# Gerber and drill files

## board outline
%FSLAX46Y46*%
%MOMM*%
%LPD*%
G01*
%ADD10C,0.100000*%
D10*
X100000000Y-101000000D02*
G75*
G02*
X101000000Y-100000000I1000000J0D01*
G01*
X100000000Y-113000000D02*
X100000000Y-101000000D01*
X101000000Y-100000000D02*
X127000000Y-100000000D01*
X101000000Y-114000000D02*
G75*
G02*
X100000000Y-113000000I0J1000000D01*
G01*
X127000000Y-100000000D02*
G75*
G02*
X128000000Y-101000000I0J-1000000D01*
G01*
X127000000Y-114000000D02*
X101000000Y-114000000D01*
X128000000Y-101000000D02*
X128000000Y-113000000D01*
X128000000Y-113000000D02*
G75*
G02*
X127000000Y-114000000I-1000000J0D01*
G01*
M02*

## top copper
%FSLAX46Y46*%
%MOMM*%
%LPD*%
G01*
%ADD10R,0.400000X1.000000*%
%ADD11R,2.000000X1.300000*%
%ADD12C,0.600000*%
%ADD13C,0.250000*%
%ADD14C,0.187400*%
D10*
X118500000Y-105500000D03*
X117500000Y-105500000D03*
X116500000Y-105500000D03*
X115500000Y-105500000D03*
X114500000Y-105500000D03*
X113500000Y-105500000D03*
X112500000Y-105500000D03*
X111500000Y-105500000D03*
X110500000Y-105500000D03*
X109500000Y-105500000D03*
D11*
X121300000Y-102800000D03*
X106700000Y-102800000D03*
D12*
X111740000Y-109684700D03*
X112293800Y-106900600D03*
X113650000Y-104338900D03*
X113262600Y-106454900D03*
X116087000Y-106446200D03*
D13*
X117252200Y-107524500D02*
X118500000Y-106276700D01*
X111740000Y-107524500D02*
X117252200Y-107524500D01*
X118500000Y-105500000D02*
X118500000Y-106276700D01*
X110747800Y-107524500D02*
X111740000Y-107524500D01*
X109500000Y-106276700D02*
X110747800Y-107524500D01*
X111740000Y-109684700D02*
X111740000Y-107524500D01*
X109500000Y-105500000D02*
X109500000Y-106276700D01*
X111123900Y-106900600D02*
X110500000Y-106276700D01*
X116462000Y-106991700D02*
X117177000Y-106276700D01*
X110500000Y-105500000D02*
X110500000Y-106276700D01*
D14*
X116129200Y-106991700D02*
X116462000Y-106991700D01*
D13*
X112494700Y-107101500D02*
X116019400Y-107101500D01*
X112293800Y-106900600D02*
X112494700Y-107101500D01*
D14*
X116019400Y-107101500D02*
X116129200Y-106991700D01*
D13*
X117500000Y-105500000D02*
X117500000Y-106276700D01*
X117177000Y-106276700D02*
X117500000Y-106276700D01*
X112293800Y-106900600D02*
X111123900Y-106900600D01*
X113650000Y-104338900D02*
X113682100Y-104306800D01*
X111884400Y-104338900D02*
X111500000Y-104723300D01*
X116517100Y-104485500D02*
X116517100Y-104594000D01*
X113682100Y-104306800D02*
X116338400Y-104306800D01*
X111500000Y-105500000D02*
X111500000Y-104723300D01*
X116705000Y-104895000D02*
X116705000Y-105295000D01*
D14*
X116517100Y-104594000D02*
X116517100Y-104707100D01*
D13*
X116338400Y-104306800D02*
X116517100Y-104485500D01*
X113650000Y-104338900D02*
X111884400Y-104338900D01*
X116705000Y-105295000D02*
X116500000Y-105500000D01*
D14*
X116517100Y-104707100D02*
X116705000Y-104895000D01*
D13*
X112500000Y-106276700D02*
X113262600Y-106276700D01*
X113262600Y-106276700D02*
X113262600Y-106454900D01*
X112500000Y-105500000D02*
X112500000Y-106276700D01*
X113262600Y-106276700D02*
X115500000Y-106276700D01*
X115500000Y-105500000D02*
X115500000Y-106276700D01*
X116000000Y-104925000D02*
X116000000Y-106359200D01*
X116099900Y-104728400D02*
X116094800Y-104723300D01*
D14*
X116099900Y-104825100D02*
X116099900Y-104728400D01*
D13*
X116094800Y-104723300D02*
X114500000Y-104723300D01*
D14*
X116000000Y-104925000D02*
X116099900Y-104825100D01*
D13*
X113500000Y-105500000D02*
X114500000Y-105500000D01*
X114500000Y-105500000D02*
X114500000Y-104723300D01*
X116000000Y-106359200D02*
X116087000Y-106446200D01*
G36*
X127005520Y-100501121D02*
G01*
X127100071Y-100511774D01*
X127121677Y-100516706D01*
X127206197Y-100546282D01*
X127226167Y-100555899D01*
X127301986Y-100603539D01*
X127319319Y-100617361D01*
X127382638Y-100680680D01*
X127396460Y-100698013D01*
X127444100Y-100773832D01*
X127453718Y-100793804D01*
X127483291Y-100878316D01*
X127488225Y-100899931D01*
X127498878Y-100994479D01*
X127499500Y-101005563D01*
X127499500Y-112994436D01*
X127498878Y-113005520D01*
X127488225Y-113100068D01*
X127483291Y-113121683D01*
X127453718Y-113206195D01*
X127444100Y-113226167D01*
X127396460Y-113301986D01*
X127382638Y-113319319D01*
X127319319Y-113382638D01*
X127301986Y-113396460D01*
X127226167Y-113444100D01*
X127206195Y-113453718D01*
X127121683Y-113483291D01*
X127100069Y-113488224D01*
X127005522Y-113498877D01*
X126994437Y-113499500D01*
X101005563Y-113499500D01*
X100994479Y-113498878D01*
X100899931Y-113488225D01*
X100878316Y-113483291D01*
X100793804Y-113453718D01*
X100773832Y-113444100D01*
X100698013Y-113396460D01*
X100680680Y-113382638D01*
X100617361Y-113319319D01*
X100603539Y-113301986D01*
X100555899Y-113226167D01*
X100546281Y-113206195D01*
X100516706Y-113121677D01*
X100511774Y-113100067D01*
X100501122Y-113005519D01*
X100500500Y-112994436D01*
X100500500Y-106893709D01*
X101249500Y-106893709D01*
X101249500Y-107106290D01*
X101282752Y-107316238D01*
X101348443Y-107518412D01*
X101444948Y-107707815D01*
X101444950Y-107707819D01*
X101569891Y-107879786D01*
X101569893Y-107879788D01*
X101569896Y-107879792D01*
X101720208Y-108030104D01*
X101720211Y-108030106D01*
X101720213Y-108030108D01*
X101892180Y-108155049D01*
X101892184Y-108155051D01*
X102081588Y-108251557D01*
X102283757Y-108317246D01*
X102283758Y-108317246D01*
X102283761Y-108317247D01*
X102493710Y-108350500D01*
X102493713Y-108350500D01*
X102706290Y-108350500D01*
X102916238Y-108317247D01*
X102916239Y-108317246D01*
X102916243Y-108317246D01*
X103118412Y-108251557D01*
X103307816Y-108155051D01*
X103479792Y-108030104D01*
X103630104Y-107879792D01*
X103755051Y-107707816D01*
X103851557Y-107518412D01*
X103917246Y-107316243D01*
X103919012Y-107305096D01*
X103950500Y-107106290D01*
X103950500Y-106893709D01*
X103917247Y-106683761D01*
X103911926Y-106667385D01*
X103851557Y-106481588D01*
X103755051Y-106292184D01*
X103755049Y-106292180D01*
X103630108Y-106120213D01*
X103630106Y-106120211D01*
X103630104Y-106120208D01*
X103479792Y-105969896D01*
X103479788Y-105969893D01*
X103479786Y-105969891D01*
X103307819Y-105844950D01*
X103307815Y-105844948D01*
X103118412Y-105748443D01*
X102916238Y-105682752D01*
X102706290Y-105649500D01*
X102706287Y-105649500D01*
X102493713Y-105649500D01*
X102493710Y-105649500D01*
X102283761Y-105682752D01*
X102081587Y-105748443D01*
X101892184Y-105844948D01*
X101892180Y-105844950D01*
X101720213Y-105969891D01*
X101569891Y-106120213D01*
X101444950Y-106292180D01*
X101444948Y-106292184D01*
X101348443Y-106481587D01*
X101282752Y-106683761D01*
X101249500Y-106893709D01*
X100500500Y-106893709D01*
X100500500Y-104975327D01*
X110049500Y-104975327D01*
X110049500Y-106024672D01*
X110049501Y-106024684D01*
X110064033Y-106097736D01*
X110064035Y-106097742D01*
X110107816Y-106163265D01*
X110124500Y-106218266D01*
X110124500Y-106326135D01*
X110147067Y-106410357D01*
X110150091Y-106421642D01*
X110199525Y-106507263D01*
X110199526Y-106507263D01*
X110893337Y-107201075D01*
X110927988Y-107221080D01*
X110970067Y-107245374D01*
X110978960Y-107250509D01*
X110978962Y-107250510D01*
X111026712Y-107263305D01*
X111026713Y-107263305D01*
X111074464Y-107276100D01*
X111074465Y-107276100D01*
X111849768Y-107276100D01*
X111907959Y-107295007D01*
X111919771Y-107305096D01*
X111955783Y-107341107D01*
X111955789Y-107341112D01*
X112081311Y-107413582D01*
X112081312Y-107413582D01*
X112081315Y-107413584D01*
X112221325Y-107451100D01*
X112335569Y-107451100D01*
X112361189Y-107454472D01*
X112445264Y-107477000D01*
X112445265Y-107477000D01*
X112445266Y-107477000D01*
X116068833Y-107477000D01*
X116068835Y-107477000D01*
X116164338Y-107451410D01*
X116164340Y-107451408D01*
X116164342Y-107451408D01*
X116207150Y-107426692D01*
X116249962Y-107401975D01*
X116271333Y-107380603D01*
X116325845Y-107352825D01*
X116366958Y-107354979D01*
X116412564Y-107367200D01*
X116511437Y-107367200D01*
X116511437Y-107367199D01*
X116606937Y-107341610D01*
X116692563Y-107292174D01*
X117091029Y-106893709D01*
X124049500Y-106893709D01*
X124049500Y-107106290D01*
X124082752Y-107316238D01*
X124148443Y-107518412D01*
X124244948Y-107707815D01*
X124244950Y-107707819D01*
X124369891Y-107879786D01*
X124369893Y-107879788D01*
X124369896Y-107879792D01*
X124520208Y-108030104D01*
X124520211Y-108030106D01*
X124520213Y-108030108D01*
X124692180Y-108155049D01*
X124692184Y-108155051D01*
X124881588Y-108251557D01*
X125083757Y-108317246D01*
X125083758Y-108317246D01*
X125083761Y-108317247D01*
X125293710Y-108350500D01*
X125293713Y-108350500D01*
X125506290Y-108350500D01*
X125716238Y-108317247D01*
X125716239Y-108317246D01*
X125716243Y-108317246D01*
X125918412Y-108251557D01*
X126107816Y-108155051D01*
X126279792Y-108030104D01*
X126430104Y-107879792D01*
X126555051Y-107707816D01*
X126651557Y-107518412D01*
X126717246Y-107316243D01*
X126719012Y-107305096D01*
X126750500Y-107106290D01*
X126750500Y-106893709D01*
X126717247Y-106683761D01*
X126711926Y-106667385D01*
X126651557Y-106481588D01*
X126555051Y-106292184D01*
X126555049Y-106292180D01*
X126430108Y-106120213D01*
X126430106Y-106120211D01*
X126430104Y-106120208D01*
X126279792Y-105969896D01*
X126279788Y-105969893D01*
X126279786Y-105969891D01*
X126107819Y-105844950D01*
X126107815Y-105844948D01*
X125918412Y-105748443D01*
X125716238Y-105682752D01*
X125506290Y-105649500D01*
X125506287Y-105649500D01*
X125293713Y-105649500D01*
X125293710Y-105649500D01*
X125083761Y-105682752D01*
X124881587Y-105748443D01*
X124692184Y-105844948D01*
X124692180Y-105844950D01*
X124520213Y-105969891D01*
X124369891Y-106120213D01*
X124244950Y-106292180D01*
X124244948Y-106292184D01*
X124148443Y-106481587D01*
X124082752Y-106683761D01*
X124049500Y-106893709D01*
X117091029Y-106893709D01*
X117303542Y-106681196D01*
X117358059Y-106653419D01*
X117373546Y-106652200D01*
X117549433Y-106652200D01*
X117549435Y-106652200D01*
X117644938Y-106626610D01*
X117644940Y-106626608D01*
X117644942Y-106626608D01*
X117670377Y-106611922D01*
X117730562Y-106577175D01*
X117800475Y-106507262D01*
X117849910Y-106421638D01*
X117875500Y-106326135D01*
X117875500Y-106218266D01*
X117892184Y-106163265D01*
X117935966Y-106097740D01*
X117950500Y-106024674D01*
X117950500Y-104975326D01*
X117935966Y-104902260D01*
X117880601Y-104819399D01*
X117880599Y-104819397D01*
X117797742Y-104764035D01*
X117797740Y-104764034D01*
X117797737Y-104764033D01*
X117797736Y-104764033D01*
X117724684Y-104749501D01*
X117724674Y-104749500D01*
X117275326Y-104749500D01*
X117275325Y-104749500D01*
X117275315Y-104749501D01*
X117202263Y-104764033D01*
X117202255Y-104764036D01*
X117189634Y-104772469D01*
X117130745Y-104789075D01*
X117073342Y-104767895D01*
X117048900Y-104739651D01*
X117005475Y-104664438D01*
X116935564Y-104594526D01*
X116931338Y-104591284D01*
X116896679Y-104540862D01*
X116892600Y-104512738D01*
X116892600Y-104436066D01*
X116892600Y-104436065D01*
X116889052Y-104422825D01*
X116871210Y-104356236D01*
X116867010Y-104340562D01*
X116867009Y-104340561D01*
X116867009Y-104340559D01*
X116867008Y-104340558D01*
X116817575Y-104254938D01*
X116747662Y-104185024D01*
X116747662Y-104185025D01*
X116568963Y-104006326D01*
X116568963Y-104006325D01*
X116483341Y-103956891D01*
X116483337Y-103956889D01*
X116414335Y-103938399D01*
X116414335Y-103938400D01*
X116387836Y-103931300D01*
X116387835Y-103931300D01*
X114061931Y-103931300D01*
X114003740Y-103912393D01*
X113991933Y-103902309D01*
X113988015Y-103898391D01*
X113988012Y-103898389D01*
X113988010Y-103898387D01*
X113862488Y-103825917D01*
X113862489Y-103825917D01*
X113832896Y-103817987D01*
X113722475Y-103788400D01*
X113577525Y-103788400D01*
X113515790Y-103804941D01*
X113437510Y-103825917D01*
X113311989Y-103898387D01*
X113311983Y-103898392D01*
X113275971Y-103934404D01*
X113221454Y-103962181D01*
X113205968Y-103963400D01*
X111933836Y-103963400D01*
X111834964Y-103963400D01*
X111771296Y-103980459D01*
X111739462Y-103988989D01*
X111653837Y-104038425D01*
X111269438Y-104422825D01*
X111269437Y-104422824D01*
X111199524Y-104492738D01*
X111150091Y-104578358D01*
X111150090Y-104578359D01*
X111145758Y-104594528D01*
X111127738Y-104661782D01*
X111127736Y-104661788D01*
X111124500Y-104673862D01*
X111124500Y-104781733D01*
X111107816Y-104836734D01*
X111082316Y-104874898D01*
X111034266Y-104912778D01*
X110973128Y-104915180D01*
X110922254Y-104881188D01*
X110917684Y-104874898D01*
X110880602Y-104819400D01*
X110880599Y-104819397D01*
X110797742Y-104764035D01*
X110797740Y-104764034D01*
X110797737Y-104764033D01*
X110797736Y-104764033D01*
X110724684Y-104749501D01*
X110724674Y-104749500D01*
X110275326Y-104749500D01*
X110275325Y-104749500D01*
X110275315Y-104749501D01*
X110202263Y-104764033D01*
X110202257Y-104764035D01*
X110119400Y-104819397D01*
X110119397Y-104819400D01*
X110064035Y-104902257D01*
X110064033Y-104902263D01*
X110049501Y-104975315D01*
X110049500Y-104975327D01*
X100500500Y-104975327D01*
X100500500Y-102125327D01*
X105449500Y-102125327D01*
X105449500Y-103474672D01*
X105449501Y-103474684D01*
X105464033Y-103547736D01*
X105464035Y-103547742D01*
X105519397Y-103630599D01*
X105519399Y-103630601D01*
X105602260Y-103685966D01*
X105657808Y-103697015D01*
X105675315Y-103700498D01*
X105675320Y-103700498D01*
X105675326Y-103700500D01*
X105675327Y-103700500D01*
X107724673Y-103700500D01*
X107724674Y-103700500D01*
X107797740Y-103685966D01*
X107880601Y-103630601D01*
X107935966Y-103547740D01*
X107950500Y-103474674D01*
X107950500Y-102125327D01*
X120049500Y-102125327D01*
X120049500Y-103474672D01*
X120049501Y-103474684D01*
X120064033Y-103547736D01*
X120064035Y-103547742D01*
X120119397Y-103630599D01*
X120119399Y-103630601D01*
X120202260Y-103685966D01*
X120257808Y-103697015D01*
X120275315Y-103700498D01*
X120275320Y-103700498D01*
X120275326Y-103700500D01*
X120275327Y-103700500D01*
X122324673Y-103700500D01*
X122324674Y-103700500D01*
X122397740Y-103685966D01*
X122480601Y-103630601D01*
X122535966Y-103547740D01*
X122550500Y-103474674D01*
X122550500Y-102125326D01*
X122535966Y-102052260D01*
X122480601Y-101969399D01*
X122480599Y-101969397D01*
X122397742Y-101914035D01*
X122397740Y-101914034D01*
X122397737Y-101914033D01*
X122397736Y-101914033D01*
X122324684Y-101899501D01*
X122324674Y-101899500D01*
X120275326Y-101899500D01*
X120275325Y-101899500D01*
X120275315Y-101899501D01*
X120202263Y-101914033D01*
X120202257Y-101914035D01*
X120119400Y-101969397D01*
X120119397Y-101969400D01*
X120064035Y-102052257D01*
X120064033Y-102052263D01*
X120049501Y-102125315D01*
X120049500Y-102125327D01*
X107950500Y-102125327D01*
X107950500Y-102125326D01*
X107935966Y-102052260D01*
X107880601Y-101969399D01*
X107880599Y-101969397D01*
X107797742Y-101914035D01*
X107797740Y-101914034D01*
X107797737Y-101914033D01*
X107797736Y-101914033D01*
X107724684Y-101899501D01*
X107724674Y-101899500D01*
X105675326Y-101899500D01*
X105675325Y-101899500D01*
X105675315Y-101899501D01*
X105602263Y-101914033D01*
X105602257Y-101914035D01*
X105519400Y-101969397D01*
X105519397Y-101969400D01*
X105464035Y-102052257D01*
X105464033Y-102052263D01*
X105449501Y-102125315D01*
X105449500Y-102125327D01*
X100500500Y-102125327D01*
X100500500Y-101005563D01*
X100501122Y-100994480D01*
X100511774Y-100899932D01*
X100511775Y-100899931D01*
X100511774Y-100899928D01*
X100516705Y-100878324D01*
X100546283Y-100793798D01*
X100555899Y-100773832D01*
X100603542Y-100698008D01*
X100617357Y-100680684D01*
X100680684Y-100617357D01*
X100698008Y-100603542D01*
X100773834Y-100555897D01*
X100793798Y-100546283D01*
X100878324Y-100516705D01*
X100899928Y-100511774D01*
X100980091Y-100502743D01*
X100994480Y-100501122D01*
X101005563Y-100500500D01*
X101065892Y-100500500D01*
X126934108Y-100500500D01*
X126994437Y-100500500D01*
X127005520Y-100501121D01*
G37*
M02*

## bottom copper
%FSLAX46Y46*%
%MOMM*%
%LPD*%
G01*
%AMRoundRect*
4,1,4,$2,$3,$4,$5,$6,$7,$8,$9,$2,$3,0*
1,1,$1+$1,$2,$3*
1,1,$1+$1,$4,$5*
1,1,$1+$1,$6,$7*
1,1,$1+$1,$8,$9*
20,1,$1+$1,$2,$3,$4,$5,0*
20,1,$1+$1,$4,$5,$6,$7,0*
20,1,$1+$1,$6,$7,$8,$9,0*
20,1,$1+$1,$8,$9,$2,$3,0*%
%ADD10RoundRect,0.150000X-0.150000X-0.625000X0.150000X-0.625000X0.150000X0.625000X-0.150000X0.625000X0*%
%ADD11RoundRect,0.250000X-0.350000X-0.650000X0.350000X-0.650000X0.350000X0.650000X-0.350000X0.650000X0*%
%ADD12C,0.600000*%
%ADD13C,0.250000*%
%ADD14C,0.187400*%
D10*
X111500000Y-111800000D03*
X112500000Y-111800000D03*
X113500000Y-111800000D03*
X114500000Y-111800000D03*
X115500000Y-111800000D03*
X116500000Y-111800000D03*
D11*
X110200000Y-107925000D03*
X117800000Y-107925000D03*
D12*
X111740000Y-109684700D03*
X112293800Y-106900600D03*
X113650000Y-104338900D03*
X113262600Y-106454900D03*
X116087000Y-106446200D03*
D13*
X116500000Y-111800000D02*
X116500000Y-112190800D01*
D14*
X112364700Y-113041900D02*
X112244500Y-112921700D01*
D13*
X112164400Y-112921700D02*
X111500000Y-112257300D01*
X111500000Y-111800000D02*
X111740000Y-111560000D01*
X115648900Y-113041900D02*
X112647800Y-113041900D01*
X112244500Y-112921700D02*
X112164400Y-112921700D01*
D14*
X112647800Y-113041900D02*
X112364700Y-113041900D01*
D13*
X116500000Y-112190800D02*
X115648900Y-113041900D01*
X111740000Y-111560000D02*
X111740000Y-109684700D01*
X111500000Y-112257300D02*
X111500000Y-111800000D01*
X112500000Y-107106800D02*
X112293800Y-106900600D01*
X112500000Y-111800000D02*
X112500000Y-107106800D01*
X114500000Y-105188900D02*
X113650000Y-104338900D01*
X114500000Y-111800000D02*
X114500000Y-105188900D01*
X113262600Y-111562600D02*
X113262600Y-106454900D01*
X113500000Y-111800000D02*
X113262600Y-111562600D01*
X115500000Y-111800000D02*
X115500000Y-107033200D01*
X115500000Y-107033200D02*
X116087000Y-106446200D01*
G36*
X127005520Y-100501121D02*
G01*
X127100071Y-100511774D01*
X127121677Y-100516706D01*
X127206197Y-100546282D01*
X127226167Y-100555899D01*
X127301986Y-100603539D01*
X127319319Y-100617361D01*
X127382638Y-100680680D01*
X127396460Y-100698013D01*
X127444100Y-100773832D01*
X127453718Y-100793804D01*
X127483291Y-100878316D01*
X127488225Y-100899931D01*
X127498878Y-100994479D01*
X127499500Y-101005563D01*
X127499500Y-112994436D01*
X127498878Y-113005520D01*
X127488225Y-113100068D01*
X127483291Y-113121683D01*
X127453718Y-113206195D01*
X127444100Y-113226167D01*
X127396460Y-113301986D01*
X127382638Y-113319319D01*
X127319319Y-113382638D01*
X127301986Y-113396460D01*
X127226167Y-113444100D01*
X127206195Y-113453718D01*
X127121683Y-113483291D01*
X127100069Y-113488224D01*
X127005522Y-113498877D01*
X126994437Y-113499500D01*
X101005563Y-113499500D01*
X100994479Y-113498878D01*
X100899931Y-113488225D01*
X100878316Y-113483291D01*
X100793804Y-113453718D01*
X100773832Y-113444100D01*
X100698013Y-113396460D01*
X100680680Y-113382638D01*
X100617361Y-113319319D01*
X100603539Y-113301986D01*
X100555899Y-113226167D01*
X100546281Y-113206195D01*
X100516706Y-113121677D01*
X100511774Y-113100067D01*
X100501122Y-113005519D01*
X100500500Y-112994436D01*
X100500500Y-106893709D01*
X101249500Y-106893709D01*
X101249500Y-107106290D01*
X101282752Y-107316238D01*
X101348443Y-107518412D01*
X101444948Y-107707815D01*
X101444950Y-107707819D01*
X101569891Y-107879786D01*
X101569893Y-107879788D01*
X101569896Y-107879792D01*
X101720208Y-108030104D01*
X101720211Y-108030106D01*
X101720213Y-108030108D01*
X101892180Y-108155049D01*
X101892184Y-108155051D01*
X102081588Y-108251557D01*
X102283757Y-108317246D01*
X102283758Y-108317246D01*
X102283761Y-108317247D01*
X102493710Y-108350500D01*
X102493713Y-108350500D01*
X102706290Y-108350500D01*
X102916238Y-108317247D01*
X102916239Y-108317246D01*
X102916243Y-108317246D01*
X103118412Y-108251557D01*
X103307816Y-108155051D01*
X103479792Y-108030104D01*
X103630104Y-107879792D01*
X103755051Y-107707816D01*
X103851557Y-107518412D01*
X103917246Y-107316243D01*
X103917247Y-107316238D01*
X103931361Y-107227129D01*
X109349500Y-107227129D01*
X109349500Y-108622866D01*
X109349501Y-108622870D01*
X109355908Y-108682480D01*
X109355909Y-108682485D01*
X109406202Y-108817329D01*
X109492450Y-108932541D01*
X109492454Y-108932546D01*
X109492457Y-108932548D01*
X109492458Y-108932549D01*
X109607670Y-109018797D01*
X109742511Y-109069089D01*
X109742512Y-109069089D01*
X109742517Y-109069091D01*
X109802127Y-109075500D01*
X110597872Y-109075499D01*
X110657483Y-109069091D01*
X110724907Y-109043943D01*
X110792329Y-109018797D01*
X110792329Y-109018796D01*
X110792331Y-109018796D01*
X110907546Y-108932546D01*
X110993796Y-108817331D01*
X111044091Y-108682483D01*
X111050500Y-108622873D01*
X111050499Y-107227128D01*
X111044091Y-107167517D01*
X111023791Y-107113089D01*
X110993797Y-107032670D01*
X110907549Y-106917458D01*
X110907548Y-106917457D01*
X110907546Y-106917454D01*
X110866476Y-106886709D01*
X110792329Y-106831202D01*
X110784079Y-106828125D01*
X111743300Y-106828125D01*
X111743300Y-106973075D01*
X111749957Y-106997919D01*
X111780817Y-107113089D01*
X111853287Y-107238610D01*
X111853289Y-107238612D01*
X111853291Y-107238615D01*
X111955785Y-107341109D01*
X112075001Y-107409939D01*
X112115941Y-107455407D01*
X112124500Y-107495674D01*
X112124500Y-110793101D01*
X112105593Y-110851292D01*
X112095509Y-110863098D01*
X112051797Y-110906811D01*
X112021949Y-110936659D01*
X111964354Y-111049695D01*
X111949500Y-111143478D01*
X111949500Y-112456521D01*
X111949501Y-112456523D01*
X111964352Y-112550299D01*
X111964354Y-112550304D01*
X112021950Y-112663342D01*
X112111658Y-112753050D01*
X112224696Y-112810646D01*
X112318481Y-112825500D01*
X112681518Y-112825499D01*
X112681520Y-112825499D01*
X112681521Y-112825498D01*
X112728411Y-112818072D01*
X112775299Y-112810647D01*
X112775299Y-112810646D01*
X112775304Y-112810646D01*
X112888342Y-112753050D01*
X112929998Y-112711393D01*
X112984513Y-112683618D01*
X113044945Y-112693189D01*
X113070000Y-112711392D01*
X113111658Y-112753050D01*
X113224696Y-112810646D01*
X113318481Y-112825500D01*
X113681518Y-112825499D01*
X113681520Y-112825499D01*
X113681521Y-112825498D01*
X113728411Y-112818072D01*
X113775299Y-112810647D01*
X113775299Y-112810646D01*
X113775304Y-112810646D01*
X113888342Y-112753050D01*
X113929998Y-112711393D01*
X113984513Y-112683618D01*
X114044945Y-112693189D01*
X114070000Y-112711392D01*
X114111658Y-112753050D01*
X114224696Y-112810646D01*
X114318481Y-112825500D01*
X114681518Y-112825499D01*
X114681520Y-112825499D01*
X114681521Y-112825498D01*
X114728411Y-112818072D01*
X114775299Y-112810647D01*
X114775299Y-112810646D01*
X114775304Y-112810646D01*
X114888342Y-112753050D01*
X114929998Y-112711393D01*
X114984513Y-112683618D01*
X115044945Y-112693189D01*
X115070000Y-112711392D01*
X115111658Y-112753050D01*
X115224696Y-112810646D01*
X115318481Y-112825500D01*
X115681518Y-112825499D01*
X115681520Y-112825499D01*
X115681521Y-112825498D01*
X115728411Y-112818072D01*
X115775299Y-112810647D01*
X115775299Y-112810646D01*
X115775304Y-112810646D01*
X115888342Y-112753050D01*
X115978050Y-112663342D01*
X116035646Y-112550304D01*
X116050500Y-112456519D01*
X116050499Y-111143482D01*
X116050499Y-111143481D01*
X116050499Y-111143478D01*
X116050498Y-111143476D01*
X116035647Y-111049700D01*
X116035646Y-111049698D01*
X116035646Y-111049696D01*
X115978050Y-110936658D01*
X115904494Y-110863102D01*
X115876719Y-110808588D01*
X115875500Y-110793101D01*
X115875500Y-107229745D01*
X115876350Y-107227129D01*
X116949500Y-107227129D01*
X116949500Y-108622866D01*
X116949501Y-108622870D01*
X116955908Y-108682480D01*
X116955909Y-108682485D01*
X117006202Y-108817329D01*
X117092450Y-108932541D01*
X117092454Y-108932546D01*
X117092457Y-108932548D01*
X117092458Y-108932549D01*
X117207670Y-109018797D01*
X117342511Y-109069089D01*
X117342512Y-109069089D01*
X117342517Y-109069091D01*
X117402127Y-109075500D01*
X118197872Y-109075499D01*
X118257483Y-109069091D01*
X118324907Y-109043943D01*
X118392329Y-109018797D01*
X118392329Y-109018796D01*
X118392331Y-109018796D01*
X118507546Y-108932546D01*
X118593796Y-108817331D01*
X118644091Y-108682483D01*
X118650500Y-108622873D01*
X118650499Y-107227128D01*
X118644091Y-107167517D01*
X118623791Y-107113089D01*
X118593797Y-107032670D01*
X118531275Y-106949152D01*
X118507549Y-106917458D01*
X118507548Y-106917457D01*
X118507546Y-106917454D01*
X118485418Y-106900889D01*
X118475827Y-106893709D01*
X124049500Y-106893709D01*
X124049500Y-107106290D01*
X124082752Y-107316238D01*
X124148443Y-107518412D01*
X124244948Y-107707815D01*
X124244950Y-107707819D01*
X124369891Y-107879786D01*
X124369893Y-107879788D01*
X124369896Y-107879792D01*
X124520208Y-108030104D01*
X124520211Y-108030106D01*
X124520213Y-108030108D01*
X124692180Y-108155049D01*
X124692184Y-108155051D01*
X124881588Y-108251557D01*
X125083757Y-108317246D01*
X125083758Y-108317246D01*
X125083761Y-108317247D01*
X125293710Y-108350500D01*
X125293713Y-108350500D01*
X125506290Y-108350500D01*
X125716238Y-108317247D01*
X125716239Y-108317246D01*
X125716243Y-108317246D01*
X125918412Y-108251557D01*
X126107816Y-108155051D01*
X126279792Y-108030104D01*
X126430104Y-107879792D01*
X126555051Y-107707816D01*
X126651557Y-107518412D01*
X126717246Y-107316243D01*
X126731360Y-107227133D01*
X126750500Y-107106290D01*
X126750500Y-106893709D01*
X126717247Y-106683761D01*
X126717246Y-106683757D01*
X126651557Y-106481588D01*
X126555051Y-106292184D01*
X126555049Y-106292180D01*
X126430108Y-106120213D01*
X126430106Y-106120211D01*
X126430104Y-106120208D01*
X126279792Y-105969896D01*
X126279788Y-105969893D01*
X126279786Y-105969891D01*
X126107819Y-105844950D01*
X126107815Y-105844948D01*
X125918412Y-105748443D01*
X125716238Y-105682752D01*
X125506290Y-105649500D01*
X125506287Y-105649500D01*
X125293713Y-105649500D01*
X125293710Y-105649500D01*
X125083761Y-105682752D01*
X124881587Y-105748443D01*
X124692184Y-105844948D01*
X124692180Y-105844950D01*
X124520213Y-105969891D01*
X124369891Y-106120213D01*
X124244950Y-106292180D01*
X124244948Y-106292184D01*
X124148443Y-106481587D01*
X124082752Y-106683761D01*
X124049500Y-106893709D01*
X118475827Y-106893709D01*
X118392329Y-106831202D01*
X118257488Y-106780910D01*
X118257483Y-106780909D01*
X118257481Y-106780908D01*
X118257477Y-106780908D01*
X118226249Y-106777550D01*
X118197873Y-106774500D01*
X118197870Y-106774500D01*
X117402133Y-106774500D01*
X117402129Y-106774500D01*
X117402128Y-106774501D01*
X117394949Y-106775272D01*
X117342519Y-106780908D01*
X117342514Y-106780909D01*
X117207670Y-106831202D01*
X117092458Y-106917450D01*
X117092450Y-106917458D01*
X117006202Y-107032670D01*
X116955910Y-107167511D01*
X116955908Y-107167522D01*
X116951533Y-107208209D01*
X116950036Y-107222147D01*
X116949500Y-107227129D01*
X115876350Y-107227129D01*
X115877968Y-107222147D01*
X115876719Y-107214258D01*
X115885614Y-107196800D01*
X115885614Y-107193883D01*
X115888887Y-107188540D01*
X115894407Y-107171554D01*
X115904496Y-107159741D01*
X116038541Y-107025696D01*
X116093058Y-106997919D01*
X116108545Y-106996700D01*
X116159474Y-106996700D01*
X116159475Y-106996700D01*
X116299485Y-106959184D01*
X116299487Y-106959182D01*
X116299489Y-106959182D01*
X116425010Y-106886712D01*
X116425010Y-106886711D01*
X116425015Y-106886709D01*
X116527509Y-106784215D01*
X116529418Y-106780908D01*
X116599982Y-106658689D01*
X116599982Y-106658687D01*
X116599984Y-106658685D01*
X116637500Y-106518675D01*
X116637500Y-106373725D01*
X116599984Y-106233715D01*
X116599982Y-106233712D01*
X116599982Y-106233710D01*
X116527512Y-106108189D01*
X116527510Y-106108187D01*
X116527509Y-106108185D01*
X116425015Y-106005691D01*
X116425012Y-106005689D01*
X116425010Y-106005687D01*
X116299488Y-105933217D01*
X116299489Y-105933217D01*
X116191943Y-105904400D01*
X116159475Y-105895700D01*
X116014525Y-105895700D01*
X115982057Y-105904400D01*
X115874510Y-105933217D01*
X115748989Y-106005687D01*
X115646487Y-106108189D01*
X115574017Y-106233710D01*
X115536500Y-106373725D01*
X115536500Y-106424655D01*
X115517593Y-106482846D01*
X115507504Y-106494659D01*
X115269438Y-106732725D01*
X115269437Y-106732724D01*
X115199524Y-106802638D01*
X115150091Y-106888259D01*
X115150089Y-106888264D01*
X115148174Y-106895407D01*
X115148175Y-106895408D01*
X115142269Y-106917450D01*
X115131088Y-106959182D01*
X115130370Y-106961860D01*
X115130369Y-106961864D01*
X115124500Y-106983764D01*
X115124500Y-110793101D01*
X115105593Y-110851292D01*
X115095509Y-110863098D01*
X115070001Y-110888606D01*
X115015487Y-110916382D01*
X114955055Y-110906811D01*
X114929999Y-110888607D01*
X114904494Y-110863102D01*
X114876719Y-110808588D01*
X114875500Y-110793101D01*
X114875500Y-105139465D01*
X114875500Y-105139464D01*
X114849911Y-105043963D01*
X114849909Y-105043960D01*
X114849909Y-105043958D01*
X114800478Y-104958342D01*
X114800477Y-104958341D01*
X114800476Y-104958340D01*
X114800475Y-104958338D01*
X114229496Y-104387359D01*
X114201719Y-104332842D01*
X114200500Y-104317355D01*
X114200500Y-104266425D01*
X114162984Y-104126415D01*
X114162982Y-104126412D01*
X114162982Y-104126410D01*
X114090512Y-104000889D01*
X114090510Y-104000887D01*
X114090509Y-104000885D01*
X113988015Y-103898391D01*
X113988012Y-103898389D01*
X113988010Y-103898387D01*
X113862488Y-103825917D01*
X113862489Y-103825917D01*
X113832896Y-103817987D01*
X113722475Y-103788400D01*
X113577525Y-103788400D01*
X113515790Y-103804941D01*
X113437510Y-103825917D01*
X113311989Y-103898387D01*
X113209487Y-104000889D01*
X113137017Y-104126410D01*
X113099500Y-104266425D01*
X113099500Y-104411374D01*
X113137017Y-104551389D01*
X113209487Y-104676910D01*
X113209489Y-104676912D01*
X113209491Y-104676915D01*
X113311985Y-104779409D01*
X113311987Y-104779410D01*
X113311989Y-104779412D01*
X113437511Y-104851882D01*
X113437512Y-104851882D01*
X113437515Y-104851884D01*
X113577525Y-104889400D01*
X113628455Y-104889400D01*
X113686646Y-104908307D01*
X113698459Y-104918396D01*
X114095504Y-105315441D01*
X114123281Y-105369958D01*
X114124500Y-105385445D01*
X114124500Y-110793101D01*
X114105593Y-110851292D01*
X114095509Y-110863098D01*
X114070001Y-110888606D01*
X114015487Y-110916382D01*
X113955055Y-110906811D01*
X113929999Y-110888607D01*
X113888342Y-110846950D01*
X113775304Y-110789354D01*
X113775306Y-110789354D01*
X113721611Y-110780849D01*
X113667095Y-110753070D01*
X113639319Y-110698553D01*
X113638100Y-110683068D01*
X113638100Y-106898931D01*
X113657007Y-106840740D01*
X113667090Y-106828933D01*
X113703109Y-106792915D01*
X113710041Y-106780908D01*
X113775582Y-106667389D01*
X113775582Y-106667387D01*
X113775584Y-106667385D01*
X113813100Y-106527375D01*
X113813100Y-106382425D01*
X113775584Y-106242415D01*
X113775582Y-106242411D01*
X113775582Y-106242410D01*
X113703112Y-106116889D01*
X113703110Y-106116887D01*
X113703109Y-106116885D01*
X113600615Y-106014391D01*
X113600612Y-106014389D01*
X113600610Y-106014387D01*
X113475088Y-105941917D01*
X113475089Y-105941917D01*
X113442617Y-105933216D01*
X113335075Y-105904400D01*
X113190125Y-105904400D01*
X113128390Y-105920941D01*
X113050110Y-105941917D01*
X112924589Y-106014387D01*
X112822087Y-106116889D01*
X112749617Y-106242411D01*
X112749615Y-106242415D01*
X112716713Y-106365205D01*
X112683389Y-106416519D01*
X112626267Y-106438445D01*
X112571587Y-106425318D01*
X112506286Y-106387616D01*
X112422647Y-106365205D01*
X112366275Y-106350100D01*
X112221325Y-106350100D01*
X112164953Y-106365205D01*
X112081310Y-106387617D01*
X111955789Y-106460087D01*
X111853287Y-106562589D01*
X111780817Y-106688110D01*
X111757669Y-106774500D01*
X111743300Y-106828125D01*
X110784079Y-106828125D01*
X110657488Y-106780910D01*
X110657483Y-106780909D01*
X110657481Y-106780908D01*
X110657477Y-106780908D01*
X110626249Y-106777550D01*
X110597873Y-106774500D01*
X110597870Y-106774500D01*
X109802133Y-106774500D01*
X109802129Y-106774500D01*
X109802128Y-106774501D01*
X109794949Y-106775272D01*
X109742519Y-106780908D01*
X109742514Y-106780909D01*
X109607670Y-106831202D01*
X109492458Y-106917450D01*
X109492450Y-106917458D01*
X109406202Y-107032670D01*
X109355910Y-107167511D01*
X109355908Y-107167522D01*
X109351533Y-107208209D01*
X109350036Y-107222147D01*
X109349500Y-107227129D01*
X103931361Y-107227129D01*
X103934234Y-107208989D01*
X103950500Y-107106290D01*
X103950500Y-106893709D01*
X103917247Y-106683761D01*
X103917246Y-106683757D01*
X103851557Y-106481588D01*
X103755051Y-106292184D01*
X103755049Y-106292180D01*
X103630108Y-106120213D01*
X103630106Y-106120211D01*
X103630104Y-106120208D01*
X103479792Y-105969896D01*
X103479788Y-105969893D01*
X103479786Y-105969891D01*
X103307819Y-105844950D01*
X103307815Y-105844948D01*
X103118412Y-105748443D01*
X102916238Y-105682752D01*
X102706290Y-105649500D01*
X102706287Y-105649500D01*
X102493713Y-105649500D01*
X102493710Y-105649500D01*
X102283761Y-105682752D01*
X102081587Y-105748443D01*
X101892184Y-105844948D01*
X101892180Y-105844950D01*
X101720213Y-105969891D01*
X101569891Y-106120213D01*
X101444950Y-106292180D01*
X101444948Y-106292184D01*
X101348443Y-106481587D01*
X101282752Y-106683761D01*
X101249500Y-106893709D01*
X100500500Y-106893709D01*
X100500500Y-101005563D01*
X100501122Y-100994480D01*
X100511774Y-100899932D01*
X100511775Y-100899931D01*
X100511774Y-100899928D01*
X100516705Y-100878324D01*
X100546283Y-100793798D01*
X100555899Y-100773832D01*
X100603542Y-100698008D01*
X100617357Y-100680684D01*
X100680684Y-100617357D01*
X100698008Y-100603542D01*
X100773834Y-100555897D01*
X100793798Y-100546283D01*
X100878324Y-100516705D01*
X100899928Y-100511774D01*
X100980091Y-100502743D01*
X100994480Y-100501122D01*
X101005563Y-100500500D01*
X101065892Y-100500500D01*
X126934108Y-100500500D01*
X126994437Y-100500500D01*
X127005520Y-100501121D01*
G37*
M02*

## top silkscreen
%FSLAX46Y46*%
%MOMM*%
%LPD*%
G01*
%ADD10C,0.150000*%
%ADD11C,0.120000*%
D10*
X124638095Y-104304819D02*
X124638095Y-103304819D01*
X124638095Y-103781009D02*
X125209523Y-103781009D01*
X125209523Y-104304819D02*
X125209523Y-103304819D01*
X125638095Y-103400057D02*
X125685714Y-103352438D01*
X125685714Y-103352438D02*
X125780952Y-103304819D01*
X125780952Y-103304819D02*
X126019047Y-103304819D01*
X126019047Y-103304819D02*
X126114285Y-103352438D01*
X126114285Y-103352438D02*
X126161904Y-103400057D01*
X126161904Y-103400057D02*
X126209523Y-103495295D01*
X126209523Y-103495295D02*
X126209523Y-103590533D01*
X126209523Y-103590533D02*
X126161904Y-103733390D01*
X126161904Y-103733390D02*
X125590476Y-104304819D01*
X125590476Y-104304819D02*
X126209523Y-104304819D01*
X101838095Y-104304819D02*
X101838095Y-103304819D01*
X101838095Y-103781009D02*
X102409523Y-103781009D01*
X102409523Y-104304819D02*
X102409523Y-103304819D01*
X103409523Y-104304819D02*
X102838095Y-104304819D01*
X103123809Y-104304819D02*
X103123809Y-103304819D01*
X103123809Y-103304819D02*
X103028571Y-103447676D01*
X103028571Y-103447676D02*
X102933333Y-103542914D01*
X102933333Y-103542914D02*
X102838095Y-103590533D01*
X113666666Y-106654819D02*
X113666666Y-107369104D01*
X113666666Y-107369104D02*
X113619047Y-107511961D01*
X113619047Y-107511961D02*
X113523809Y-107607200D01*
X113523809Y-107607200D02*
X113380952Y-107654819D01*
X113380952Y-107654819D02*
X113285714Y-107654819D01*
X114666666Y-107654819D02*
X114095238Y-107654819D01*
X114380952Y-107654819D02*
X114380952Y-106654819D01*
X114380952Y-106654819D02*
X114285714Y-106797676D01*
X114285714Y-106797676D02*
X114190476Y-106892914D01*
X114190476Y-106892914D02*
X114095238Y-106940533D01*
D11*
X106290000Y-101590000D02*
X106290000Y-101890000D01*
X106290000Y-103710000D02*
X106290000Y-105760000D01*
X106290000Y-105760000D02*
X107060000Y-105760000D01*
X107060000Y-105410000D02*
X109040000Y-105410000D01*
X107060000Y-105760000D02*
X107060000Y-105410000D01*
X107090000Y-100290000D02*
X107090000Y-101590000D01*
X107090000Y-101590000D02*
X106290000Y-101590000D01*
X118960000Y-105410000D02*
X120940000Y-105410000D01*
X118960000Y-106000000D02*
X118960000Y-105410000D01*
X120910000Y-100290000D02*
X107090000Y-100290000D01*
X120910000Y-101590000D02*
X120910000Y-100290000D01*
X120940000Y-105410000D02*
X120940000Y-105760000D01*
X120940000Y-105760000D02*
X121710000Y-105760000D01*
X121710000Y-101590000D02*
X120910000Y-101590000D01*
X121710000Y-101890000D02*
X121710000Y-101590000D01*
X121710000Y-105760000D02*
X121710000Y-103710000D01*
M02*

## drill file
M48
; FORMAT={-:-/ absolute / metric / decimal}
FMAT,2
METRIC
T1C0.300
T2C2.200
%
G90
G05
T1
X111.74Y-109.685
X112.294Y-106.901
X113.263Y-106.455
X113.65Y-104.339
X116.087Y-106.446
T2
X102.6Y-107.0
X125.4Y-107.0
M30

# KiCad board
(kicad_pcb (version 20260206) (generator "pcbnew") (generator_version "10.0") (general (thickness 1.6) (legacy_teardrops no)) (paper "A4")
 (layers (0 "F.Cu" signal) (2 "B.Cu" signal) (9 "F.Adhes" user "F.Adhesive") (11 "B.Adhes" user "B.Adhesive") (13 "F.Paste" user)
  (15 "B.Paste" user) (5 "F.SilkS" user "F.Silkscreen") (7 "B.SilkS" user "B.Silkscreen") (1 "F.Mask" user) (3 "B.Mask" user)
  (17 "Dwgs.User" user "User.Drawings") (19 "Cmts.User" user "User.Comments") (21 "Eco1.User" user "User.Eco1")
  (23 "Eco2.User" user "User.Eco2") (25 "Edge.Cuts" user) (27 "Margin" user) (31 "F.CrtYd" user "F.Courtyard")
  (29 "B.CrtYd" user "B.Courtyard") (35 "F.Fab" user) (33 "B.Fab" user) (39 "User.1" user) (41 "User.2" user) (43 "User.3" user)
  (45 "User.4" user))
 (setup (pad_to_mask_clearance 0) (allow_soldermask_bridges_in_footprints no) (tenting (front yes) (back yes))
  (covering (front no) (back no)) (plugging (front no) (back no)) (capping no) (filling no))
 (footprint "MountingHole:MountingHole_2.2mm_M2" (layer "F.Cu") (at 125.4 107)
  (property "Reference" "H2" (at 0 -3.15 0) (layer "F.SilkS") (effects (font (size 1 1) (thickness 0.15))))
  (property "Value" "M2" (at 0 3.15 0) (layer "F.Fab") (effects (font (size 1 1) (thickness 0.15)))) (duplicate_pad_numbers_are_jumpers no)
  (pad "" np_thru_hole circle (at 0 0) (size 2.2 2.2) (drill 2.2) (layers "*.Cu" "*.Mask") (zone_connect 2)))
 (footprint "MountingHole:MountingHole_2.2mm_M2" (layer "F.Cu") (at 102.6 107)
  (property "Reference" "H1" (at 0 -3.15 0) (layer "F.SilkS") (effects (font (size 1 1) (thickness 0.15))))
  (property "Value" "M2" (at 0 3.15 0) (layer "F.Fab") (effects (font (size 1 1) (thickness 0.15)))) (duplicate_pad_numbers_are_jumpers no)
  (pad "" np_thru_hole circle (at 0 0) (size 2.2 2.2) (drill 2.2) (layers "*.Cu" "*.Mask") (zone_connect 2)))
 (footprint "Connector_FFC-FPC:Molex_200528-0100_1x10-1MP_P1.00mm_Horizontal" (layer "F.Cu") (at 114 104.59 180)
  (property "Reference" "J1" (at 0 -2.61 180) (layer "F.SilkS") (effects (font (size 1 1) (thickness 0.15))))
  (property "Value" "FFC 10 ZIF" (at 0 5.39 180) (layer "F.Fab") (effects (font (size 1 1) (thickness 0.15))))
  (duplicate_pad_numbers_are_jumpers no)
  (fp_line (start 7.71 3) (end 7.71 2.7) (stroke (width 0.12) (type solid)) (layer "F.SilkS"))
  (fp_line (start 7.71 0.88) (end 7.71 -1.17) (stroke (width 0.12) (type solid)) (layer "F.SilkS"))
  (fp_line (start 7.71 -1.17) (end 6.94 -1.17) (stroke (width 0.12) (type solid)) (layer "F.SilkS"))
  (fp_line (start 6.94 -0.82) (end 4.96 -0.82) (stroke (width 0.12) (type solid)) (layer "F.SilkS"))
  (fp_line (start 6.94 -1.17) (end 6.94 -0.82) (stroke (width 0.12) (type solid)) (layer "F.SilkS"))
  (fp_line (start 6.91 4.3) (end 6.91 3) (stroke (width 0.12) (type solid)) (layer "F.SilkS"))
  (fp_line (start 6.91 3) (end 7.71 3) (stroke (width 0.12) (type solid)) (layer "F.SilkS"))
  (fp_line (start -4.96 -0.82) (end -6.94 -0.82) (stroke (width 0.12) (type solid)) (layer "F.SilkS"))
  (fp_line (start -4.96 -1.41) (end -4.96 -0.82) (stroke (width 0.12) (type solid)) (layer "F.SilkS"))
  (fp_line (start -6.91 4.3) (end 6.91 4.3) (stroke (width 0.12) (type solid)) (layer "F.SilkS"))
  (fp_line (start -6.91 3) (end -6.91 4.3) (stroke (width 0.12) (type solid)) (layer "F.SilkS"))
  (fp_line (start -6.94 -0.82) (end -6.94 -1.17) (stroke (width 0.12) (type solid)) (layer "F.SilkS"))
  (fp_line (start -6.94 -1.17) (end -7.71 -1.17) (stroke (width 0.12) (type solid)) (layer "F.SilkS"))
  (fp_line (start -7.71 3) (end -6.91 3) (stroke (width 0.12) (type solid)) (layer "F.SilkS"))
  (fp_line (start -7.71 2.7) (end -7.71 3) (stroke (width 0.12) (type solid)) (layer "F.SilkS"))
  (fp_line (start -7.71 -1.17) (end -7.71 0.88) (stroke (width 0.12) (type solid)) (layer "F.SilkS"))
  (pad "1" smd rect (at -4.5 -0.91 180) (size 0.4 1) (layers "F.Cu" "F.Mask" "F.Paste") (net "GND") (zone_connect 2))
  (pad "2" smd rect (at -3.5 -0.91 180) (size 0.4 1) (layers "F.Cu" "F.Mask" "F.Paste") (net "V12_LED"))
  (pad "3" smd rect (at -2.5 -0.91 180) (size 0.4 1) (layers "F.Cu" "F.Mask" "F.Paste") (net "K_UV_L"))
  (pad "4" smd rect (at -1.5 -0.91 180) (size 0.4 1) (layers "F.Cu" "F.Mask" "F.Paste") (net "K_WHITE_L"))
  (pad "5" smd rect (at -0.5 -0.91 180) (size 0.4 1) (layers "F.Cu" "F.Mask" "F.Paste") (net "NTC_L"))
  (pad "6" smd rect (at 0.5 -0.91 180) (size 0.4 1) (layers "F.Cu" "F.Mask" "F.Paste") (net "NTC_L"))
  (pad "7" smd rect (at 1.5 -0.91 180) (size 0.4 1) (layers "F.Cu" "F.Mask" "F.Paste") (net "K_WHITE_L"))
  (pad "8" smd rect (at 2.5 -0.91 180) (size 0.4 1) (layers "F.Cu" "F.Mask" "F.Paste") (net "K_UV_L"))
  (pad "9" smd rect (at 3.5 -0.91 180) (size 0.4 1) (layers "F.Cu" "F.Mask" "F.Paste") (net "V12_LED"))
  (pad "10" smd rect (at 4.5 -0.91 180) (size 0.4 1) (layers "F.Cu" "F.Mask" "F.Paste") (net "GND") (zone_connect 2))
  (pad "MP" smd rect (at -7.3 1.79 180) (size 2 1.3) (layers "F.Cu" "F.Mask" "F.Paste") (zone_connect 2))
  (pad "MP" smd rect (at 7.3 1.79 180) (size 2 1.3) (layers "F.Cu" "F.Mask" "F.Paste") (zone_connect 2)))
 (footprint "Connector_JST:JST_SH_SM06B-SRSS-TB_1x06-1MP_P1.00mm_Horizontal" (layer "B.Cu") (at 114 109.8)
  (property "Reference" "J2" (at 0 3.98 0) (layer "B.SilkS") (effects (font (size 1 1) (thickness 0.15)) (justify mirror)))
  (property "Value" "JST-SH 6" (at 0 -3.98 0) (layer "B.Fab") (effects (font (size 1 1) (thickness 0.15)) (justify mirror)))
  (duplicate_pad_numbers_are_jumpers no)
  (pad "1" smd roundrect (at -2.5 2) (size 0.6 1.55) (layers "B.Cu" "B.Mask" "B.Paste") (roundrect_rratio 0.25) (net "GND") (zone_connect 2))
  (pad "2" smd roundrect (at -1.5 2) (size 0.6 1.55) (layers "B.Cu" "B.Mask" "B.Paste") (roundrect_rratio 0.25) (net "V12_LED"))
  (pad "3" smd roundrect (at -0.5 2) (size 0.6 1.55) (layers "B.Cu" "B.Mask" "B.Paste") (roundrect_rratio 0.25) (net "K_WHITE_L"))
  (pad "4" smd roundrect (at 0.5 2) (size 0.6 1.55) (layers "B.Cu" "B.Mask" "B.Paste") (roundrect_rratio 0.25) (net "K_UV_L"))
  (pad "5" smd roundrect (at 1.5 2) (size 0.6 1.55) (layers "B.Cu" "B.Mask" "B.Paste") (roundrect_rratio 0.25) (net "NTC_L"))
  (pad "6" smd roundrect (at 2.5 2) (size 0.6 1.55) (layers "B.Cu" "B.Mask" "B.Paste") (roundrect_rratio 0.25) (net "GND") (zone_connect 2))
  (pad "MP" smd roundrect (at -3.8 -1.875) (size 1.2 1.8) (layers "B.Cu" "B.Mask" "B.Paste") (roundrect_rratio 0.208333) (zone_connect 2))
  (pad "MP" smd roundrect (at 3.8 -1.875) (size 1.2 1.8) (layers "B.Cu" "B.Mask" "B.Paste") (roundrect_rratio 0.208333) (zone_connect 2)))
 (gr_arc (start 100 101) (mid 100.292893 100.292893) (end 101 100) (stroke (width 0.1) (type default)) (layer "Edge.Cuts"))
 (gr_line (start 100 113) (end 100 101) (stroke (width 0.1) (type default)) (layer "Edge.Cuts"))
 (gr_line (start 101 100) (end 127 100) (stroke (width 0.1) (type default)) (layer "Edge.Cuts"))
 (gr_arc (start 101 114) (mid 100.292893 113.707107) (end 100 113) (stroke (width 0.1) (type default)) (layer "Edge.Cuts"))
 (gr_arc (start 127 100) (mid 127.707107 100.292893) (end 128 101) (stroke (width 0.1) (type default)) (layer "Edge.Cuts"))
 (gr_line (start 127 114) (end 101 114) (stroke (width 0.1) (type default)) (layer "Edge.Cuts"))
 (gr_line (start 128 101) (end 128 113) (stroke (width 0.1) (type default)) (layer "Edge.Cuts"))
 (gr_arc (start 128 113) (mid 127.707107 113.707107) (end 127 114) (stroke (width 0.1) (type default)) (layer "Edge.Cuts"))
 (segment (start 117.2522 107.5245) (end 118.5 106.2767) (width 0.25) (layer "F.Cu") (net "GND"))
 (segment (start 111.74 107.5245) (end 117.2522 107.5245) (width 0.25) (layer "F.Cu") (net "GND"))
 (segment (start 118.5 105.5) (end 118.5 106.2767) (width 0.25) (layer "F.Cu") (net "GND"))
 (segment (start 110.7478 107.5245) (end 111.74 107.5245) (width 0.25) (layer "F.Cu") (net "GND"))
 (segment (start 109.5 106.2767) (end 110.7478 107.5245) (width 0.25) (layer "F.Cu") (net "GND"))
 (segment (start 111.74 109.6847) (end 111.74 107.5245) (width 0.25) (layer "F.Cu") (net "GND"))
 (segment (start 109.5 105.5) (end 109.5 106.2767) (width 0.25) (layer "F.Cu") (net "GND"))
 (via (at 111.74 109.6847) (size 0.6) (drill 0.3) (layers "F.Cu" "B.Cu") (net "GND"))
 (segment (start 116.5 111.8) (end 116.5 112.1908) (width 0.25) (layer "B.Cu") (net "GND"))
 (segment (start 112.3647 113.0419) (end 112.2445 112.9217) (width 0.1874) (layer "B.Cu") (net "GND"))
 (segment (start 112.1644 112.9217) (end 111.5 112.2573) (width 0.25) (layer "B.Cu") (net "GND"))
 (segment (start 111.5 111.8) (end 111.74 111.56) (width 0.25) (layer "B.Cu") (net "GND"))
 (segment (start 115.6489 113.0419) (end 112.6478 113.0419) (width 0.25) (layer "B.Cu") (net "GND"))
 (segment (start 112.2445 112.9217) (end 112.1644 112.9217) (width 0.25) (layer "B.Cu") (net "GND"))
 (segment (start 112.6478 113.0419) (end 112.3647 113.0419) (width 0.1874) (layer "B.Cu") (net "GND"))
 (segment (start 116.5 112.1908) (end 115.6489 113.0419) (width 0.25) (layer "B.Cu") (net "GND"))
 (segment (start 111.74 111.56) (end 111.74 109.6847) (width 0.25) (layer "B.Cu") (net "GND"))
 (segment (start 111.5 112.2573) (end 111.5 111.8) (width 0.25) (layer "B.Cu") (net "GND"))
 (segment (start 111.1239 106.9006) (end 110.5 106.2767) (width 0.25) (layer "F.Cu") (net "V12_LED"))
 (segment (start 116.462 106.9917) (end 117.177 106.2767) (width 0.25) (layer "F.Cu") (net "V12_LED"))
 (segment (start 110.5 105.5) (end 110.5 106.2767) (width 0.25) (layer "F.Cu") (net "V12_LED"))
 (segment (start 116.1292 106.9917) (end 116.462 106.9917) (width 0.1874) (layer "F.Cu") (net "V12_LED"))
 (segment (start 112.4947 107.1015) (end 116.0194 107.1015) (width 0.25) (layer "F.Cu") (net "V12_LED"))
 (segment (start 112.2938 106.9006) (end 112.4947 107.1015) (width 0.25) (layer "F.Cu") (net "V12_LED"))
 (segment (start 116.0194 107.1015) (end 116.1292 106.9917) (width 0.1874) (layer "F.Cu") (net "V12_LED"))
 (segment (start 117.5 105.5) (end 117.5 106.2767) (width 0.25) (layer "F.Cu") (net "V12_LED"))
 (segment (start 117.177 106.2767) (end 117.5 106.2767) (width 0.25) (layer "F.Cu") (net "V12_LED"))
 (segment (start 112.2938 106.9006) (end 111.1239 106.9006) (width 0.25) (layer "F.Cu") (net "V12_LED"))
 (via (at 112.2938 106.9006) (size 0.6) (drill 0.3) (layers "F.Cu" "B.Cu") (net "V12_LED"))
 (segment (start 112.5 107.1068) (end 112.2938 106.9006) (width 0.25) (layer "B.Cu") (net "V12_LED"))
 (segment (start 112.5 111.8) (end 112.5 107.1068) (width 0.25) (layer "B.Cu") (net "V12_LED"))
 (segment (start 113.65 104.3389) (end 113.6821 104.3068) (width 0.25) (layer "F.Cu") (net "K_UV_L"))
 (segment (start 111.8844 104.3389) (end 111.5 104.7233) (width 0.25) (layer "F.Cu") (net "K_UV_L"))
 (segment (start 116.5171 104.4855) (end 116.5171 104.594) (width 0.25) (layer "F.Cu") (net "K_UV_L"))
 (segment (start 113.6821 104.3068) (end 116.3384 104.3068) (width 0.25) (layer "F.Cu") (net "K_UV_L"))
 (segment (start 111.5 105.5) (end 111.5 104.7233) (width 0.25) (layer "F.Cu") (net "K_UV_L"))
 (segment (start 116.705 104.895) (end 116.705 105.295) (width 0.25) (layer "F.Cu") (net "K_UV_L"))
 (segment (start 116.5171 104.594) (end 116.5171 104.7071) (width 0.1874) (layer "F.Cu") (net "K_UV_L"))
 (segment (start 116.3384 104.3068) (end 116.5171 104.4855) (width 0.25) (layer "F.Cu") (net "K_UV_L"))
 (segment (start 113.65 104.3389) (end 111.8844 104.3389) (width 0.25) (layer "F.Cu") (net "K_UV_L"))
 (segment (start 116.705 105.295) (end 116.5 105.5) (width 0.25) (layer "F.Cu") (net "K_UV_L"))
 (segment (start 116.5171 104.7071) (end 116.705 104.895) (width 0.1874) (layer "F.Cu") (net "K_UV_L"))
 (via (at 113.65 104.3389) (size 0.6) (drill 0.3) (layers "F.Cu" "B.Cu") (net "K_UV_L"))
 (segment (start 114.5 105.1889) (end 113.65 104.3389) (width 0.25) (layer "B.Cu") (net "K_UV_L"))
 (segment (start 114.5 111.8) (end 114.5 105.1889) (width 0.25) (layer "B.Cu") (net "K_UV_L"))
 (segment (start 112.5 106.2767) (end 113.2626 106.2767) (width 0.25) (layer "F.Cu") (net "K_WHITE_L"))
 (segment (start 113.2626 106.2767) (end 113.2626 106.4549) (width 0.25) (layer "F.Cu") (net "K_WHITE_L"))
 (segment (start 112.5 105.5) (end 112.5 106.2767) (width 0.25) (layer "F.Cu") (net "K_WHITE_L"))
 (segment (start 113.2626 106.2767) (end 115.5 106.2767) (width 0.25) (layer "F.Cu") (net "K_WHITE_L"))
 (segment (start 115.5 105.5) (end 115.5 106.2767) (width 0.25) (layer "F.Cu") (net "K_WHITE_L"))
 (via (at 113.2626 106.4549) (size 0.6) (drill 0.3) (layers "F.Cu" "B.Cu") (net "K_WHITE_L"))
 (segment (start 113.2626 111.5626) (end 113.2626 106.4549) (width 0.25) (layer "B.Cu") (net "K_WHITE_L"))
 (segment (start 113.5 111.8) (end 113.2626 111.5626) (width 0.25) (layer "B.Cu") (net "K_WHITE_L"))
 (segment (start 116 104.925) (end 116 106.3592) (width 0.25) (layer "F.Cu") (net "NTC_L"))
 (segment (start 116.0999 104.7284) (end 116.0948 104.7233) (width 0.25) (layer "F.Cu") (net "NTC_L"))
 (segment (start 116.0999 104.8251) (end 116.0999 104.7284) (width 0.1874) (layer "F.Cu") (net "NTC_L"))
 (segment (start 116.0948 104.7233) (end 114.5 104.7233) (width 0.25) (layer "F.Cu") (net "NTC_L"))
 (segment (start 116 104.925) (end 116.0999 104.8251) (width 0.1874) (layer "F.Cu") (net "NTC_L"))
 (segment (start 113.5 105.5) (end 114.5 105.5) (width 0.25) (layer "F.Cu") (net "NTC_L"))
 (segment (start 114.5 105.5) (end 114.5 104.7233) (width 0.25) (layer "F.Cu") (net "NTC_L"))
 (segment (start 116 106.3592) (end 116.087 106.4462) (width 0.25) (layer "F.Cu") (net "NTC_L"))
 (via (at 116.087 106.4462) (size 0.6) (drill 0.3) (layers "F.Cu" "B.Cu") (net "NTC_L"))
 (segment (start 115.5 111.8) (end 115.5 107.0332) (width 0.25) (layer "B.Cu") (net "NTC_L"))
 (segment (start 115.5 107.0332) (end 116.087 106.4462) (width 0.25) (layer "B.Cu") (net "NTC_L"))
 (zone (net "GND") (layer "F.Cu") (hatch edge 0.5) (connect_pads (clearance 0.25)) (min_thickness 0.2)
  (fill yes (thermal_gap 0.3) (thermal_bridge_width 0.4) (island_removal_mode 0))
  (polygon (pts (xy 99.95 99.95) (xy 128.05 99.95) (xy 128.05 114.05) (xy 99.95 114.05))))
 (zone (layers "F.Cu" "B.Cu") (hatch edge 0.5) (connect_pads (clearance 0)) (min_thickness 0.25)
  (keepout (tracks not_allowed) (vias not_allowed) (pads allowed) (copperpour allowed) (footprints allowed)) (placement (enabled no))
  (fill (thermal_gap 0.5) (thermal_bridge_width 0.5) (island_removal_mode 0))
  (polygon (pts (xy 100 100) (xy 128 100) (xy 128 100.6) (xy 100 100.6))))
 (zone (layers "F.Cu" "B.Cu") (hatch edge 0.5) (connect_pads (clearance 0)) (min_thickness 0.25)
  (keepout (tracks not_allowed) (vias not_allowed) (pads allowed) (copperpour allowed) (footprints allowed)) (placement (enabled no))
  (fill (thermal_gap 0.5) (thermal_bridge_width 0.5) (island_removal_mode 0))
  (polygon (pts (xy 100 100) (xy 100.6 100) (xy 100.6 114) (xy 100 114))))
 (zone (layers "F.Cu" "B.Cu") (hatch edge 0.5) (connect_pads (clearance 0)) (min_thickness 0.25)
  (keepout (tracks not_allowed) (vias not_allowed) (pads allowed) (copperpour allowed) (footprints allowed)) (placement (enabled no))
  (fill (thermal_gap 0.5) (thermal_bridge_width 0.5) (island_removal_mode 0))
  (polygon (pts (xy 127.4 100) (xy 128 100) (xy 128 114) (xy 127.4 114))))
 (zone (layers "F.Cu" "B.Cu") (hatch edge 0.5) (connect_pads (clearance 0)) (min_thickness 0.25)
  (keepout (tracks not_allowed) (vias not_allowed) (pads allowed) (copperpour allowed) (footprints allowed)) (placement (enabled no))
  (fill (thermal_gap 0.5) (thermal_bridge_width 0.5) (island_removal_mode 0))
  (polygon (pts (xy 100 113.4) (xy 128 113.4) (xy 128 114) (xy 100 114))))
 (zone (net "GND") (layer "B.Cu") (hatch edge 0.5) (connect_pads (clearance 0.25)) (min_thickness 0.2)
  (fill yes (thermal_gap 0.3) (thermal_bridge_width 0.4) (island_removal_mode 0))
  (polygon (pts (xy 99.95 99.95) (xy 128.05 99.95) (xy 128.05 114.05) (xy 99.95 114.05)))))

